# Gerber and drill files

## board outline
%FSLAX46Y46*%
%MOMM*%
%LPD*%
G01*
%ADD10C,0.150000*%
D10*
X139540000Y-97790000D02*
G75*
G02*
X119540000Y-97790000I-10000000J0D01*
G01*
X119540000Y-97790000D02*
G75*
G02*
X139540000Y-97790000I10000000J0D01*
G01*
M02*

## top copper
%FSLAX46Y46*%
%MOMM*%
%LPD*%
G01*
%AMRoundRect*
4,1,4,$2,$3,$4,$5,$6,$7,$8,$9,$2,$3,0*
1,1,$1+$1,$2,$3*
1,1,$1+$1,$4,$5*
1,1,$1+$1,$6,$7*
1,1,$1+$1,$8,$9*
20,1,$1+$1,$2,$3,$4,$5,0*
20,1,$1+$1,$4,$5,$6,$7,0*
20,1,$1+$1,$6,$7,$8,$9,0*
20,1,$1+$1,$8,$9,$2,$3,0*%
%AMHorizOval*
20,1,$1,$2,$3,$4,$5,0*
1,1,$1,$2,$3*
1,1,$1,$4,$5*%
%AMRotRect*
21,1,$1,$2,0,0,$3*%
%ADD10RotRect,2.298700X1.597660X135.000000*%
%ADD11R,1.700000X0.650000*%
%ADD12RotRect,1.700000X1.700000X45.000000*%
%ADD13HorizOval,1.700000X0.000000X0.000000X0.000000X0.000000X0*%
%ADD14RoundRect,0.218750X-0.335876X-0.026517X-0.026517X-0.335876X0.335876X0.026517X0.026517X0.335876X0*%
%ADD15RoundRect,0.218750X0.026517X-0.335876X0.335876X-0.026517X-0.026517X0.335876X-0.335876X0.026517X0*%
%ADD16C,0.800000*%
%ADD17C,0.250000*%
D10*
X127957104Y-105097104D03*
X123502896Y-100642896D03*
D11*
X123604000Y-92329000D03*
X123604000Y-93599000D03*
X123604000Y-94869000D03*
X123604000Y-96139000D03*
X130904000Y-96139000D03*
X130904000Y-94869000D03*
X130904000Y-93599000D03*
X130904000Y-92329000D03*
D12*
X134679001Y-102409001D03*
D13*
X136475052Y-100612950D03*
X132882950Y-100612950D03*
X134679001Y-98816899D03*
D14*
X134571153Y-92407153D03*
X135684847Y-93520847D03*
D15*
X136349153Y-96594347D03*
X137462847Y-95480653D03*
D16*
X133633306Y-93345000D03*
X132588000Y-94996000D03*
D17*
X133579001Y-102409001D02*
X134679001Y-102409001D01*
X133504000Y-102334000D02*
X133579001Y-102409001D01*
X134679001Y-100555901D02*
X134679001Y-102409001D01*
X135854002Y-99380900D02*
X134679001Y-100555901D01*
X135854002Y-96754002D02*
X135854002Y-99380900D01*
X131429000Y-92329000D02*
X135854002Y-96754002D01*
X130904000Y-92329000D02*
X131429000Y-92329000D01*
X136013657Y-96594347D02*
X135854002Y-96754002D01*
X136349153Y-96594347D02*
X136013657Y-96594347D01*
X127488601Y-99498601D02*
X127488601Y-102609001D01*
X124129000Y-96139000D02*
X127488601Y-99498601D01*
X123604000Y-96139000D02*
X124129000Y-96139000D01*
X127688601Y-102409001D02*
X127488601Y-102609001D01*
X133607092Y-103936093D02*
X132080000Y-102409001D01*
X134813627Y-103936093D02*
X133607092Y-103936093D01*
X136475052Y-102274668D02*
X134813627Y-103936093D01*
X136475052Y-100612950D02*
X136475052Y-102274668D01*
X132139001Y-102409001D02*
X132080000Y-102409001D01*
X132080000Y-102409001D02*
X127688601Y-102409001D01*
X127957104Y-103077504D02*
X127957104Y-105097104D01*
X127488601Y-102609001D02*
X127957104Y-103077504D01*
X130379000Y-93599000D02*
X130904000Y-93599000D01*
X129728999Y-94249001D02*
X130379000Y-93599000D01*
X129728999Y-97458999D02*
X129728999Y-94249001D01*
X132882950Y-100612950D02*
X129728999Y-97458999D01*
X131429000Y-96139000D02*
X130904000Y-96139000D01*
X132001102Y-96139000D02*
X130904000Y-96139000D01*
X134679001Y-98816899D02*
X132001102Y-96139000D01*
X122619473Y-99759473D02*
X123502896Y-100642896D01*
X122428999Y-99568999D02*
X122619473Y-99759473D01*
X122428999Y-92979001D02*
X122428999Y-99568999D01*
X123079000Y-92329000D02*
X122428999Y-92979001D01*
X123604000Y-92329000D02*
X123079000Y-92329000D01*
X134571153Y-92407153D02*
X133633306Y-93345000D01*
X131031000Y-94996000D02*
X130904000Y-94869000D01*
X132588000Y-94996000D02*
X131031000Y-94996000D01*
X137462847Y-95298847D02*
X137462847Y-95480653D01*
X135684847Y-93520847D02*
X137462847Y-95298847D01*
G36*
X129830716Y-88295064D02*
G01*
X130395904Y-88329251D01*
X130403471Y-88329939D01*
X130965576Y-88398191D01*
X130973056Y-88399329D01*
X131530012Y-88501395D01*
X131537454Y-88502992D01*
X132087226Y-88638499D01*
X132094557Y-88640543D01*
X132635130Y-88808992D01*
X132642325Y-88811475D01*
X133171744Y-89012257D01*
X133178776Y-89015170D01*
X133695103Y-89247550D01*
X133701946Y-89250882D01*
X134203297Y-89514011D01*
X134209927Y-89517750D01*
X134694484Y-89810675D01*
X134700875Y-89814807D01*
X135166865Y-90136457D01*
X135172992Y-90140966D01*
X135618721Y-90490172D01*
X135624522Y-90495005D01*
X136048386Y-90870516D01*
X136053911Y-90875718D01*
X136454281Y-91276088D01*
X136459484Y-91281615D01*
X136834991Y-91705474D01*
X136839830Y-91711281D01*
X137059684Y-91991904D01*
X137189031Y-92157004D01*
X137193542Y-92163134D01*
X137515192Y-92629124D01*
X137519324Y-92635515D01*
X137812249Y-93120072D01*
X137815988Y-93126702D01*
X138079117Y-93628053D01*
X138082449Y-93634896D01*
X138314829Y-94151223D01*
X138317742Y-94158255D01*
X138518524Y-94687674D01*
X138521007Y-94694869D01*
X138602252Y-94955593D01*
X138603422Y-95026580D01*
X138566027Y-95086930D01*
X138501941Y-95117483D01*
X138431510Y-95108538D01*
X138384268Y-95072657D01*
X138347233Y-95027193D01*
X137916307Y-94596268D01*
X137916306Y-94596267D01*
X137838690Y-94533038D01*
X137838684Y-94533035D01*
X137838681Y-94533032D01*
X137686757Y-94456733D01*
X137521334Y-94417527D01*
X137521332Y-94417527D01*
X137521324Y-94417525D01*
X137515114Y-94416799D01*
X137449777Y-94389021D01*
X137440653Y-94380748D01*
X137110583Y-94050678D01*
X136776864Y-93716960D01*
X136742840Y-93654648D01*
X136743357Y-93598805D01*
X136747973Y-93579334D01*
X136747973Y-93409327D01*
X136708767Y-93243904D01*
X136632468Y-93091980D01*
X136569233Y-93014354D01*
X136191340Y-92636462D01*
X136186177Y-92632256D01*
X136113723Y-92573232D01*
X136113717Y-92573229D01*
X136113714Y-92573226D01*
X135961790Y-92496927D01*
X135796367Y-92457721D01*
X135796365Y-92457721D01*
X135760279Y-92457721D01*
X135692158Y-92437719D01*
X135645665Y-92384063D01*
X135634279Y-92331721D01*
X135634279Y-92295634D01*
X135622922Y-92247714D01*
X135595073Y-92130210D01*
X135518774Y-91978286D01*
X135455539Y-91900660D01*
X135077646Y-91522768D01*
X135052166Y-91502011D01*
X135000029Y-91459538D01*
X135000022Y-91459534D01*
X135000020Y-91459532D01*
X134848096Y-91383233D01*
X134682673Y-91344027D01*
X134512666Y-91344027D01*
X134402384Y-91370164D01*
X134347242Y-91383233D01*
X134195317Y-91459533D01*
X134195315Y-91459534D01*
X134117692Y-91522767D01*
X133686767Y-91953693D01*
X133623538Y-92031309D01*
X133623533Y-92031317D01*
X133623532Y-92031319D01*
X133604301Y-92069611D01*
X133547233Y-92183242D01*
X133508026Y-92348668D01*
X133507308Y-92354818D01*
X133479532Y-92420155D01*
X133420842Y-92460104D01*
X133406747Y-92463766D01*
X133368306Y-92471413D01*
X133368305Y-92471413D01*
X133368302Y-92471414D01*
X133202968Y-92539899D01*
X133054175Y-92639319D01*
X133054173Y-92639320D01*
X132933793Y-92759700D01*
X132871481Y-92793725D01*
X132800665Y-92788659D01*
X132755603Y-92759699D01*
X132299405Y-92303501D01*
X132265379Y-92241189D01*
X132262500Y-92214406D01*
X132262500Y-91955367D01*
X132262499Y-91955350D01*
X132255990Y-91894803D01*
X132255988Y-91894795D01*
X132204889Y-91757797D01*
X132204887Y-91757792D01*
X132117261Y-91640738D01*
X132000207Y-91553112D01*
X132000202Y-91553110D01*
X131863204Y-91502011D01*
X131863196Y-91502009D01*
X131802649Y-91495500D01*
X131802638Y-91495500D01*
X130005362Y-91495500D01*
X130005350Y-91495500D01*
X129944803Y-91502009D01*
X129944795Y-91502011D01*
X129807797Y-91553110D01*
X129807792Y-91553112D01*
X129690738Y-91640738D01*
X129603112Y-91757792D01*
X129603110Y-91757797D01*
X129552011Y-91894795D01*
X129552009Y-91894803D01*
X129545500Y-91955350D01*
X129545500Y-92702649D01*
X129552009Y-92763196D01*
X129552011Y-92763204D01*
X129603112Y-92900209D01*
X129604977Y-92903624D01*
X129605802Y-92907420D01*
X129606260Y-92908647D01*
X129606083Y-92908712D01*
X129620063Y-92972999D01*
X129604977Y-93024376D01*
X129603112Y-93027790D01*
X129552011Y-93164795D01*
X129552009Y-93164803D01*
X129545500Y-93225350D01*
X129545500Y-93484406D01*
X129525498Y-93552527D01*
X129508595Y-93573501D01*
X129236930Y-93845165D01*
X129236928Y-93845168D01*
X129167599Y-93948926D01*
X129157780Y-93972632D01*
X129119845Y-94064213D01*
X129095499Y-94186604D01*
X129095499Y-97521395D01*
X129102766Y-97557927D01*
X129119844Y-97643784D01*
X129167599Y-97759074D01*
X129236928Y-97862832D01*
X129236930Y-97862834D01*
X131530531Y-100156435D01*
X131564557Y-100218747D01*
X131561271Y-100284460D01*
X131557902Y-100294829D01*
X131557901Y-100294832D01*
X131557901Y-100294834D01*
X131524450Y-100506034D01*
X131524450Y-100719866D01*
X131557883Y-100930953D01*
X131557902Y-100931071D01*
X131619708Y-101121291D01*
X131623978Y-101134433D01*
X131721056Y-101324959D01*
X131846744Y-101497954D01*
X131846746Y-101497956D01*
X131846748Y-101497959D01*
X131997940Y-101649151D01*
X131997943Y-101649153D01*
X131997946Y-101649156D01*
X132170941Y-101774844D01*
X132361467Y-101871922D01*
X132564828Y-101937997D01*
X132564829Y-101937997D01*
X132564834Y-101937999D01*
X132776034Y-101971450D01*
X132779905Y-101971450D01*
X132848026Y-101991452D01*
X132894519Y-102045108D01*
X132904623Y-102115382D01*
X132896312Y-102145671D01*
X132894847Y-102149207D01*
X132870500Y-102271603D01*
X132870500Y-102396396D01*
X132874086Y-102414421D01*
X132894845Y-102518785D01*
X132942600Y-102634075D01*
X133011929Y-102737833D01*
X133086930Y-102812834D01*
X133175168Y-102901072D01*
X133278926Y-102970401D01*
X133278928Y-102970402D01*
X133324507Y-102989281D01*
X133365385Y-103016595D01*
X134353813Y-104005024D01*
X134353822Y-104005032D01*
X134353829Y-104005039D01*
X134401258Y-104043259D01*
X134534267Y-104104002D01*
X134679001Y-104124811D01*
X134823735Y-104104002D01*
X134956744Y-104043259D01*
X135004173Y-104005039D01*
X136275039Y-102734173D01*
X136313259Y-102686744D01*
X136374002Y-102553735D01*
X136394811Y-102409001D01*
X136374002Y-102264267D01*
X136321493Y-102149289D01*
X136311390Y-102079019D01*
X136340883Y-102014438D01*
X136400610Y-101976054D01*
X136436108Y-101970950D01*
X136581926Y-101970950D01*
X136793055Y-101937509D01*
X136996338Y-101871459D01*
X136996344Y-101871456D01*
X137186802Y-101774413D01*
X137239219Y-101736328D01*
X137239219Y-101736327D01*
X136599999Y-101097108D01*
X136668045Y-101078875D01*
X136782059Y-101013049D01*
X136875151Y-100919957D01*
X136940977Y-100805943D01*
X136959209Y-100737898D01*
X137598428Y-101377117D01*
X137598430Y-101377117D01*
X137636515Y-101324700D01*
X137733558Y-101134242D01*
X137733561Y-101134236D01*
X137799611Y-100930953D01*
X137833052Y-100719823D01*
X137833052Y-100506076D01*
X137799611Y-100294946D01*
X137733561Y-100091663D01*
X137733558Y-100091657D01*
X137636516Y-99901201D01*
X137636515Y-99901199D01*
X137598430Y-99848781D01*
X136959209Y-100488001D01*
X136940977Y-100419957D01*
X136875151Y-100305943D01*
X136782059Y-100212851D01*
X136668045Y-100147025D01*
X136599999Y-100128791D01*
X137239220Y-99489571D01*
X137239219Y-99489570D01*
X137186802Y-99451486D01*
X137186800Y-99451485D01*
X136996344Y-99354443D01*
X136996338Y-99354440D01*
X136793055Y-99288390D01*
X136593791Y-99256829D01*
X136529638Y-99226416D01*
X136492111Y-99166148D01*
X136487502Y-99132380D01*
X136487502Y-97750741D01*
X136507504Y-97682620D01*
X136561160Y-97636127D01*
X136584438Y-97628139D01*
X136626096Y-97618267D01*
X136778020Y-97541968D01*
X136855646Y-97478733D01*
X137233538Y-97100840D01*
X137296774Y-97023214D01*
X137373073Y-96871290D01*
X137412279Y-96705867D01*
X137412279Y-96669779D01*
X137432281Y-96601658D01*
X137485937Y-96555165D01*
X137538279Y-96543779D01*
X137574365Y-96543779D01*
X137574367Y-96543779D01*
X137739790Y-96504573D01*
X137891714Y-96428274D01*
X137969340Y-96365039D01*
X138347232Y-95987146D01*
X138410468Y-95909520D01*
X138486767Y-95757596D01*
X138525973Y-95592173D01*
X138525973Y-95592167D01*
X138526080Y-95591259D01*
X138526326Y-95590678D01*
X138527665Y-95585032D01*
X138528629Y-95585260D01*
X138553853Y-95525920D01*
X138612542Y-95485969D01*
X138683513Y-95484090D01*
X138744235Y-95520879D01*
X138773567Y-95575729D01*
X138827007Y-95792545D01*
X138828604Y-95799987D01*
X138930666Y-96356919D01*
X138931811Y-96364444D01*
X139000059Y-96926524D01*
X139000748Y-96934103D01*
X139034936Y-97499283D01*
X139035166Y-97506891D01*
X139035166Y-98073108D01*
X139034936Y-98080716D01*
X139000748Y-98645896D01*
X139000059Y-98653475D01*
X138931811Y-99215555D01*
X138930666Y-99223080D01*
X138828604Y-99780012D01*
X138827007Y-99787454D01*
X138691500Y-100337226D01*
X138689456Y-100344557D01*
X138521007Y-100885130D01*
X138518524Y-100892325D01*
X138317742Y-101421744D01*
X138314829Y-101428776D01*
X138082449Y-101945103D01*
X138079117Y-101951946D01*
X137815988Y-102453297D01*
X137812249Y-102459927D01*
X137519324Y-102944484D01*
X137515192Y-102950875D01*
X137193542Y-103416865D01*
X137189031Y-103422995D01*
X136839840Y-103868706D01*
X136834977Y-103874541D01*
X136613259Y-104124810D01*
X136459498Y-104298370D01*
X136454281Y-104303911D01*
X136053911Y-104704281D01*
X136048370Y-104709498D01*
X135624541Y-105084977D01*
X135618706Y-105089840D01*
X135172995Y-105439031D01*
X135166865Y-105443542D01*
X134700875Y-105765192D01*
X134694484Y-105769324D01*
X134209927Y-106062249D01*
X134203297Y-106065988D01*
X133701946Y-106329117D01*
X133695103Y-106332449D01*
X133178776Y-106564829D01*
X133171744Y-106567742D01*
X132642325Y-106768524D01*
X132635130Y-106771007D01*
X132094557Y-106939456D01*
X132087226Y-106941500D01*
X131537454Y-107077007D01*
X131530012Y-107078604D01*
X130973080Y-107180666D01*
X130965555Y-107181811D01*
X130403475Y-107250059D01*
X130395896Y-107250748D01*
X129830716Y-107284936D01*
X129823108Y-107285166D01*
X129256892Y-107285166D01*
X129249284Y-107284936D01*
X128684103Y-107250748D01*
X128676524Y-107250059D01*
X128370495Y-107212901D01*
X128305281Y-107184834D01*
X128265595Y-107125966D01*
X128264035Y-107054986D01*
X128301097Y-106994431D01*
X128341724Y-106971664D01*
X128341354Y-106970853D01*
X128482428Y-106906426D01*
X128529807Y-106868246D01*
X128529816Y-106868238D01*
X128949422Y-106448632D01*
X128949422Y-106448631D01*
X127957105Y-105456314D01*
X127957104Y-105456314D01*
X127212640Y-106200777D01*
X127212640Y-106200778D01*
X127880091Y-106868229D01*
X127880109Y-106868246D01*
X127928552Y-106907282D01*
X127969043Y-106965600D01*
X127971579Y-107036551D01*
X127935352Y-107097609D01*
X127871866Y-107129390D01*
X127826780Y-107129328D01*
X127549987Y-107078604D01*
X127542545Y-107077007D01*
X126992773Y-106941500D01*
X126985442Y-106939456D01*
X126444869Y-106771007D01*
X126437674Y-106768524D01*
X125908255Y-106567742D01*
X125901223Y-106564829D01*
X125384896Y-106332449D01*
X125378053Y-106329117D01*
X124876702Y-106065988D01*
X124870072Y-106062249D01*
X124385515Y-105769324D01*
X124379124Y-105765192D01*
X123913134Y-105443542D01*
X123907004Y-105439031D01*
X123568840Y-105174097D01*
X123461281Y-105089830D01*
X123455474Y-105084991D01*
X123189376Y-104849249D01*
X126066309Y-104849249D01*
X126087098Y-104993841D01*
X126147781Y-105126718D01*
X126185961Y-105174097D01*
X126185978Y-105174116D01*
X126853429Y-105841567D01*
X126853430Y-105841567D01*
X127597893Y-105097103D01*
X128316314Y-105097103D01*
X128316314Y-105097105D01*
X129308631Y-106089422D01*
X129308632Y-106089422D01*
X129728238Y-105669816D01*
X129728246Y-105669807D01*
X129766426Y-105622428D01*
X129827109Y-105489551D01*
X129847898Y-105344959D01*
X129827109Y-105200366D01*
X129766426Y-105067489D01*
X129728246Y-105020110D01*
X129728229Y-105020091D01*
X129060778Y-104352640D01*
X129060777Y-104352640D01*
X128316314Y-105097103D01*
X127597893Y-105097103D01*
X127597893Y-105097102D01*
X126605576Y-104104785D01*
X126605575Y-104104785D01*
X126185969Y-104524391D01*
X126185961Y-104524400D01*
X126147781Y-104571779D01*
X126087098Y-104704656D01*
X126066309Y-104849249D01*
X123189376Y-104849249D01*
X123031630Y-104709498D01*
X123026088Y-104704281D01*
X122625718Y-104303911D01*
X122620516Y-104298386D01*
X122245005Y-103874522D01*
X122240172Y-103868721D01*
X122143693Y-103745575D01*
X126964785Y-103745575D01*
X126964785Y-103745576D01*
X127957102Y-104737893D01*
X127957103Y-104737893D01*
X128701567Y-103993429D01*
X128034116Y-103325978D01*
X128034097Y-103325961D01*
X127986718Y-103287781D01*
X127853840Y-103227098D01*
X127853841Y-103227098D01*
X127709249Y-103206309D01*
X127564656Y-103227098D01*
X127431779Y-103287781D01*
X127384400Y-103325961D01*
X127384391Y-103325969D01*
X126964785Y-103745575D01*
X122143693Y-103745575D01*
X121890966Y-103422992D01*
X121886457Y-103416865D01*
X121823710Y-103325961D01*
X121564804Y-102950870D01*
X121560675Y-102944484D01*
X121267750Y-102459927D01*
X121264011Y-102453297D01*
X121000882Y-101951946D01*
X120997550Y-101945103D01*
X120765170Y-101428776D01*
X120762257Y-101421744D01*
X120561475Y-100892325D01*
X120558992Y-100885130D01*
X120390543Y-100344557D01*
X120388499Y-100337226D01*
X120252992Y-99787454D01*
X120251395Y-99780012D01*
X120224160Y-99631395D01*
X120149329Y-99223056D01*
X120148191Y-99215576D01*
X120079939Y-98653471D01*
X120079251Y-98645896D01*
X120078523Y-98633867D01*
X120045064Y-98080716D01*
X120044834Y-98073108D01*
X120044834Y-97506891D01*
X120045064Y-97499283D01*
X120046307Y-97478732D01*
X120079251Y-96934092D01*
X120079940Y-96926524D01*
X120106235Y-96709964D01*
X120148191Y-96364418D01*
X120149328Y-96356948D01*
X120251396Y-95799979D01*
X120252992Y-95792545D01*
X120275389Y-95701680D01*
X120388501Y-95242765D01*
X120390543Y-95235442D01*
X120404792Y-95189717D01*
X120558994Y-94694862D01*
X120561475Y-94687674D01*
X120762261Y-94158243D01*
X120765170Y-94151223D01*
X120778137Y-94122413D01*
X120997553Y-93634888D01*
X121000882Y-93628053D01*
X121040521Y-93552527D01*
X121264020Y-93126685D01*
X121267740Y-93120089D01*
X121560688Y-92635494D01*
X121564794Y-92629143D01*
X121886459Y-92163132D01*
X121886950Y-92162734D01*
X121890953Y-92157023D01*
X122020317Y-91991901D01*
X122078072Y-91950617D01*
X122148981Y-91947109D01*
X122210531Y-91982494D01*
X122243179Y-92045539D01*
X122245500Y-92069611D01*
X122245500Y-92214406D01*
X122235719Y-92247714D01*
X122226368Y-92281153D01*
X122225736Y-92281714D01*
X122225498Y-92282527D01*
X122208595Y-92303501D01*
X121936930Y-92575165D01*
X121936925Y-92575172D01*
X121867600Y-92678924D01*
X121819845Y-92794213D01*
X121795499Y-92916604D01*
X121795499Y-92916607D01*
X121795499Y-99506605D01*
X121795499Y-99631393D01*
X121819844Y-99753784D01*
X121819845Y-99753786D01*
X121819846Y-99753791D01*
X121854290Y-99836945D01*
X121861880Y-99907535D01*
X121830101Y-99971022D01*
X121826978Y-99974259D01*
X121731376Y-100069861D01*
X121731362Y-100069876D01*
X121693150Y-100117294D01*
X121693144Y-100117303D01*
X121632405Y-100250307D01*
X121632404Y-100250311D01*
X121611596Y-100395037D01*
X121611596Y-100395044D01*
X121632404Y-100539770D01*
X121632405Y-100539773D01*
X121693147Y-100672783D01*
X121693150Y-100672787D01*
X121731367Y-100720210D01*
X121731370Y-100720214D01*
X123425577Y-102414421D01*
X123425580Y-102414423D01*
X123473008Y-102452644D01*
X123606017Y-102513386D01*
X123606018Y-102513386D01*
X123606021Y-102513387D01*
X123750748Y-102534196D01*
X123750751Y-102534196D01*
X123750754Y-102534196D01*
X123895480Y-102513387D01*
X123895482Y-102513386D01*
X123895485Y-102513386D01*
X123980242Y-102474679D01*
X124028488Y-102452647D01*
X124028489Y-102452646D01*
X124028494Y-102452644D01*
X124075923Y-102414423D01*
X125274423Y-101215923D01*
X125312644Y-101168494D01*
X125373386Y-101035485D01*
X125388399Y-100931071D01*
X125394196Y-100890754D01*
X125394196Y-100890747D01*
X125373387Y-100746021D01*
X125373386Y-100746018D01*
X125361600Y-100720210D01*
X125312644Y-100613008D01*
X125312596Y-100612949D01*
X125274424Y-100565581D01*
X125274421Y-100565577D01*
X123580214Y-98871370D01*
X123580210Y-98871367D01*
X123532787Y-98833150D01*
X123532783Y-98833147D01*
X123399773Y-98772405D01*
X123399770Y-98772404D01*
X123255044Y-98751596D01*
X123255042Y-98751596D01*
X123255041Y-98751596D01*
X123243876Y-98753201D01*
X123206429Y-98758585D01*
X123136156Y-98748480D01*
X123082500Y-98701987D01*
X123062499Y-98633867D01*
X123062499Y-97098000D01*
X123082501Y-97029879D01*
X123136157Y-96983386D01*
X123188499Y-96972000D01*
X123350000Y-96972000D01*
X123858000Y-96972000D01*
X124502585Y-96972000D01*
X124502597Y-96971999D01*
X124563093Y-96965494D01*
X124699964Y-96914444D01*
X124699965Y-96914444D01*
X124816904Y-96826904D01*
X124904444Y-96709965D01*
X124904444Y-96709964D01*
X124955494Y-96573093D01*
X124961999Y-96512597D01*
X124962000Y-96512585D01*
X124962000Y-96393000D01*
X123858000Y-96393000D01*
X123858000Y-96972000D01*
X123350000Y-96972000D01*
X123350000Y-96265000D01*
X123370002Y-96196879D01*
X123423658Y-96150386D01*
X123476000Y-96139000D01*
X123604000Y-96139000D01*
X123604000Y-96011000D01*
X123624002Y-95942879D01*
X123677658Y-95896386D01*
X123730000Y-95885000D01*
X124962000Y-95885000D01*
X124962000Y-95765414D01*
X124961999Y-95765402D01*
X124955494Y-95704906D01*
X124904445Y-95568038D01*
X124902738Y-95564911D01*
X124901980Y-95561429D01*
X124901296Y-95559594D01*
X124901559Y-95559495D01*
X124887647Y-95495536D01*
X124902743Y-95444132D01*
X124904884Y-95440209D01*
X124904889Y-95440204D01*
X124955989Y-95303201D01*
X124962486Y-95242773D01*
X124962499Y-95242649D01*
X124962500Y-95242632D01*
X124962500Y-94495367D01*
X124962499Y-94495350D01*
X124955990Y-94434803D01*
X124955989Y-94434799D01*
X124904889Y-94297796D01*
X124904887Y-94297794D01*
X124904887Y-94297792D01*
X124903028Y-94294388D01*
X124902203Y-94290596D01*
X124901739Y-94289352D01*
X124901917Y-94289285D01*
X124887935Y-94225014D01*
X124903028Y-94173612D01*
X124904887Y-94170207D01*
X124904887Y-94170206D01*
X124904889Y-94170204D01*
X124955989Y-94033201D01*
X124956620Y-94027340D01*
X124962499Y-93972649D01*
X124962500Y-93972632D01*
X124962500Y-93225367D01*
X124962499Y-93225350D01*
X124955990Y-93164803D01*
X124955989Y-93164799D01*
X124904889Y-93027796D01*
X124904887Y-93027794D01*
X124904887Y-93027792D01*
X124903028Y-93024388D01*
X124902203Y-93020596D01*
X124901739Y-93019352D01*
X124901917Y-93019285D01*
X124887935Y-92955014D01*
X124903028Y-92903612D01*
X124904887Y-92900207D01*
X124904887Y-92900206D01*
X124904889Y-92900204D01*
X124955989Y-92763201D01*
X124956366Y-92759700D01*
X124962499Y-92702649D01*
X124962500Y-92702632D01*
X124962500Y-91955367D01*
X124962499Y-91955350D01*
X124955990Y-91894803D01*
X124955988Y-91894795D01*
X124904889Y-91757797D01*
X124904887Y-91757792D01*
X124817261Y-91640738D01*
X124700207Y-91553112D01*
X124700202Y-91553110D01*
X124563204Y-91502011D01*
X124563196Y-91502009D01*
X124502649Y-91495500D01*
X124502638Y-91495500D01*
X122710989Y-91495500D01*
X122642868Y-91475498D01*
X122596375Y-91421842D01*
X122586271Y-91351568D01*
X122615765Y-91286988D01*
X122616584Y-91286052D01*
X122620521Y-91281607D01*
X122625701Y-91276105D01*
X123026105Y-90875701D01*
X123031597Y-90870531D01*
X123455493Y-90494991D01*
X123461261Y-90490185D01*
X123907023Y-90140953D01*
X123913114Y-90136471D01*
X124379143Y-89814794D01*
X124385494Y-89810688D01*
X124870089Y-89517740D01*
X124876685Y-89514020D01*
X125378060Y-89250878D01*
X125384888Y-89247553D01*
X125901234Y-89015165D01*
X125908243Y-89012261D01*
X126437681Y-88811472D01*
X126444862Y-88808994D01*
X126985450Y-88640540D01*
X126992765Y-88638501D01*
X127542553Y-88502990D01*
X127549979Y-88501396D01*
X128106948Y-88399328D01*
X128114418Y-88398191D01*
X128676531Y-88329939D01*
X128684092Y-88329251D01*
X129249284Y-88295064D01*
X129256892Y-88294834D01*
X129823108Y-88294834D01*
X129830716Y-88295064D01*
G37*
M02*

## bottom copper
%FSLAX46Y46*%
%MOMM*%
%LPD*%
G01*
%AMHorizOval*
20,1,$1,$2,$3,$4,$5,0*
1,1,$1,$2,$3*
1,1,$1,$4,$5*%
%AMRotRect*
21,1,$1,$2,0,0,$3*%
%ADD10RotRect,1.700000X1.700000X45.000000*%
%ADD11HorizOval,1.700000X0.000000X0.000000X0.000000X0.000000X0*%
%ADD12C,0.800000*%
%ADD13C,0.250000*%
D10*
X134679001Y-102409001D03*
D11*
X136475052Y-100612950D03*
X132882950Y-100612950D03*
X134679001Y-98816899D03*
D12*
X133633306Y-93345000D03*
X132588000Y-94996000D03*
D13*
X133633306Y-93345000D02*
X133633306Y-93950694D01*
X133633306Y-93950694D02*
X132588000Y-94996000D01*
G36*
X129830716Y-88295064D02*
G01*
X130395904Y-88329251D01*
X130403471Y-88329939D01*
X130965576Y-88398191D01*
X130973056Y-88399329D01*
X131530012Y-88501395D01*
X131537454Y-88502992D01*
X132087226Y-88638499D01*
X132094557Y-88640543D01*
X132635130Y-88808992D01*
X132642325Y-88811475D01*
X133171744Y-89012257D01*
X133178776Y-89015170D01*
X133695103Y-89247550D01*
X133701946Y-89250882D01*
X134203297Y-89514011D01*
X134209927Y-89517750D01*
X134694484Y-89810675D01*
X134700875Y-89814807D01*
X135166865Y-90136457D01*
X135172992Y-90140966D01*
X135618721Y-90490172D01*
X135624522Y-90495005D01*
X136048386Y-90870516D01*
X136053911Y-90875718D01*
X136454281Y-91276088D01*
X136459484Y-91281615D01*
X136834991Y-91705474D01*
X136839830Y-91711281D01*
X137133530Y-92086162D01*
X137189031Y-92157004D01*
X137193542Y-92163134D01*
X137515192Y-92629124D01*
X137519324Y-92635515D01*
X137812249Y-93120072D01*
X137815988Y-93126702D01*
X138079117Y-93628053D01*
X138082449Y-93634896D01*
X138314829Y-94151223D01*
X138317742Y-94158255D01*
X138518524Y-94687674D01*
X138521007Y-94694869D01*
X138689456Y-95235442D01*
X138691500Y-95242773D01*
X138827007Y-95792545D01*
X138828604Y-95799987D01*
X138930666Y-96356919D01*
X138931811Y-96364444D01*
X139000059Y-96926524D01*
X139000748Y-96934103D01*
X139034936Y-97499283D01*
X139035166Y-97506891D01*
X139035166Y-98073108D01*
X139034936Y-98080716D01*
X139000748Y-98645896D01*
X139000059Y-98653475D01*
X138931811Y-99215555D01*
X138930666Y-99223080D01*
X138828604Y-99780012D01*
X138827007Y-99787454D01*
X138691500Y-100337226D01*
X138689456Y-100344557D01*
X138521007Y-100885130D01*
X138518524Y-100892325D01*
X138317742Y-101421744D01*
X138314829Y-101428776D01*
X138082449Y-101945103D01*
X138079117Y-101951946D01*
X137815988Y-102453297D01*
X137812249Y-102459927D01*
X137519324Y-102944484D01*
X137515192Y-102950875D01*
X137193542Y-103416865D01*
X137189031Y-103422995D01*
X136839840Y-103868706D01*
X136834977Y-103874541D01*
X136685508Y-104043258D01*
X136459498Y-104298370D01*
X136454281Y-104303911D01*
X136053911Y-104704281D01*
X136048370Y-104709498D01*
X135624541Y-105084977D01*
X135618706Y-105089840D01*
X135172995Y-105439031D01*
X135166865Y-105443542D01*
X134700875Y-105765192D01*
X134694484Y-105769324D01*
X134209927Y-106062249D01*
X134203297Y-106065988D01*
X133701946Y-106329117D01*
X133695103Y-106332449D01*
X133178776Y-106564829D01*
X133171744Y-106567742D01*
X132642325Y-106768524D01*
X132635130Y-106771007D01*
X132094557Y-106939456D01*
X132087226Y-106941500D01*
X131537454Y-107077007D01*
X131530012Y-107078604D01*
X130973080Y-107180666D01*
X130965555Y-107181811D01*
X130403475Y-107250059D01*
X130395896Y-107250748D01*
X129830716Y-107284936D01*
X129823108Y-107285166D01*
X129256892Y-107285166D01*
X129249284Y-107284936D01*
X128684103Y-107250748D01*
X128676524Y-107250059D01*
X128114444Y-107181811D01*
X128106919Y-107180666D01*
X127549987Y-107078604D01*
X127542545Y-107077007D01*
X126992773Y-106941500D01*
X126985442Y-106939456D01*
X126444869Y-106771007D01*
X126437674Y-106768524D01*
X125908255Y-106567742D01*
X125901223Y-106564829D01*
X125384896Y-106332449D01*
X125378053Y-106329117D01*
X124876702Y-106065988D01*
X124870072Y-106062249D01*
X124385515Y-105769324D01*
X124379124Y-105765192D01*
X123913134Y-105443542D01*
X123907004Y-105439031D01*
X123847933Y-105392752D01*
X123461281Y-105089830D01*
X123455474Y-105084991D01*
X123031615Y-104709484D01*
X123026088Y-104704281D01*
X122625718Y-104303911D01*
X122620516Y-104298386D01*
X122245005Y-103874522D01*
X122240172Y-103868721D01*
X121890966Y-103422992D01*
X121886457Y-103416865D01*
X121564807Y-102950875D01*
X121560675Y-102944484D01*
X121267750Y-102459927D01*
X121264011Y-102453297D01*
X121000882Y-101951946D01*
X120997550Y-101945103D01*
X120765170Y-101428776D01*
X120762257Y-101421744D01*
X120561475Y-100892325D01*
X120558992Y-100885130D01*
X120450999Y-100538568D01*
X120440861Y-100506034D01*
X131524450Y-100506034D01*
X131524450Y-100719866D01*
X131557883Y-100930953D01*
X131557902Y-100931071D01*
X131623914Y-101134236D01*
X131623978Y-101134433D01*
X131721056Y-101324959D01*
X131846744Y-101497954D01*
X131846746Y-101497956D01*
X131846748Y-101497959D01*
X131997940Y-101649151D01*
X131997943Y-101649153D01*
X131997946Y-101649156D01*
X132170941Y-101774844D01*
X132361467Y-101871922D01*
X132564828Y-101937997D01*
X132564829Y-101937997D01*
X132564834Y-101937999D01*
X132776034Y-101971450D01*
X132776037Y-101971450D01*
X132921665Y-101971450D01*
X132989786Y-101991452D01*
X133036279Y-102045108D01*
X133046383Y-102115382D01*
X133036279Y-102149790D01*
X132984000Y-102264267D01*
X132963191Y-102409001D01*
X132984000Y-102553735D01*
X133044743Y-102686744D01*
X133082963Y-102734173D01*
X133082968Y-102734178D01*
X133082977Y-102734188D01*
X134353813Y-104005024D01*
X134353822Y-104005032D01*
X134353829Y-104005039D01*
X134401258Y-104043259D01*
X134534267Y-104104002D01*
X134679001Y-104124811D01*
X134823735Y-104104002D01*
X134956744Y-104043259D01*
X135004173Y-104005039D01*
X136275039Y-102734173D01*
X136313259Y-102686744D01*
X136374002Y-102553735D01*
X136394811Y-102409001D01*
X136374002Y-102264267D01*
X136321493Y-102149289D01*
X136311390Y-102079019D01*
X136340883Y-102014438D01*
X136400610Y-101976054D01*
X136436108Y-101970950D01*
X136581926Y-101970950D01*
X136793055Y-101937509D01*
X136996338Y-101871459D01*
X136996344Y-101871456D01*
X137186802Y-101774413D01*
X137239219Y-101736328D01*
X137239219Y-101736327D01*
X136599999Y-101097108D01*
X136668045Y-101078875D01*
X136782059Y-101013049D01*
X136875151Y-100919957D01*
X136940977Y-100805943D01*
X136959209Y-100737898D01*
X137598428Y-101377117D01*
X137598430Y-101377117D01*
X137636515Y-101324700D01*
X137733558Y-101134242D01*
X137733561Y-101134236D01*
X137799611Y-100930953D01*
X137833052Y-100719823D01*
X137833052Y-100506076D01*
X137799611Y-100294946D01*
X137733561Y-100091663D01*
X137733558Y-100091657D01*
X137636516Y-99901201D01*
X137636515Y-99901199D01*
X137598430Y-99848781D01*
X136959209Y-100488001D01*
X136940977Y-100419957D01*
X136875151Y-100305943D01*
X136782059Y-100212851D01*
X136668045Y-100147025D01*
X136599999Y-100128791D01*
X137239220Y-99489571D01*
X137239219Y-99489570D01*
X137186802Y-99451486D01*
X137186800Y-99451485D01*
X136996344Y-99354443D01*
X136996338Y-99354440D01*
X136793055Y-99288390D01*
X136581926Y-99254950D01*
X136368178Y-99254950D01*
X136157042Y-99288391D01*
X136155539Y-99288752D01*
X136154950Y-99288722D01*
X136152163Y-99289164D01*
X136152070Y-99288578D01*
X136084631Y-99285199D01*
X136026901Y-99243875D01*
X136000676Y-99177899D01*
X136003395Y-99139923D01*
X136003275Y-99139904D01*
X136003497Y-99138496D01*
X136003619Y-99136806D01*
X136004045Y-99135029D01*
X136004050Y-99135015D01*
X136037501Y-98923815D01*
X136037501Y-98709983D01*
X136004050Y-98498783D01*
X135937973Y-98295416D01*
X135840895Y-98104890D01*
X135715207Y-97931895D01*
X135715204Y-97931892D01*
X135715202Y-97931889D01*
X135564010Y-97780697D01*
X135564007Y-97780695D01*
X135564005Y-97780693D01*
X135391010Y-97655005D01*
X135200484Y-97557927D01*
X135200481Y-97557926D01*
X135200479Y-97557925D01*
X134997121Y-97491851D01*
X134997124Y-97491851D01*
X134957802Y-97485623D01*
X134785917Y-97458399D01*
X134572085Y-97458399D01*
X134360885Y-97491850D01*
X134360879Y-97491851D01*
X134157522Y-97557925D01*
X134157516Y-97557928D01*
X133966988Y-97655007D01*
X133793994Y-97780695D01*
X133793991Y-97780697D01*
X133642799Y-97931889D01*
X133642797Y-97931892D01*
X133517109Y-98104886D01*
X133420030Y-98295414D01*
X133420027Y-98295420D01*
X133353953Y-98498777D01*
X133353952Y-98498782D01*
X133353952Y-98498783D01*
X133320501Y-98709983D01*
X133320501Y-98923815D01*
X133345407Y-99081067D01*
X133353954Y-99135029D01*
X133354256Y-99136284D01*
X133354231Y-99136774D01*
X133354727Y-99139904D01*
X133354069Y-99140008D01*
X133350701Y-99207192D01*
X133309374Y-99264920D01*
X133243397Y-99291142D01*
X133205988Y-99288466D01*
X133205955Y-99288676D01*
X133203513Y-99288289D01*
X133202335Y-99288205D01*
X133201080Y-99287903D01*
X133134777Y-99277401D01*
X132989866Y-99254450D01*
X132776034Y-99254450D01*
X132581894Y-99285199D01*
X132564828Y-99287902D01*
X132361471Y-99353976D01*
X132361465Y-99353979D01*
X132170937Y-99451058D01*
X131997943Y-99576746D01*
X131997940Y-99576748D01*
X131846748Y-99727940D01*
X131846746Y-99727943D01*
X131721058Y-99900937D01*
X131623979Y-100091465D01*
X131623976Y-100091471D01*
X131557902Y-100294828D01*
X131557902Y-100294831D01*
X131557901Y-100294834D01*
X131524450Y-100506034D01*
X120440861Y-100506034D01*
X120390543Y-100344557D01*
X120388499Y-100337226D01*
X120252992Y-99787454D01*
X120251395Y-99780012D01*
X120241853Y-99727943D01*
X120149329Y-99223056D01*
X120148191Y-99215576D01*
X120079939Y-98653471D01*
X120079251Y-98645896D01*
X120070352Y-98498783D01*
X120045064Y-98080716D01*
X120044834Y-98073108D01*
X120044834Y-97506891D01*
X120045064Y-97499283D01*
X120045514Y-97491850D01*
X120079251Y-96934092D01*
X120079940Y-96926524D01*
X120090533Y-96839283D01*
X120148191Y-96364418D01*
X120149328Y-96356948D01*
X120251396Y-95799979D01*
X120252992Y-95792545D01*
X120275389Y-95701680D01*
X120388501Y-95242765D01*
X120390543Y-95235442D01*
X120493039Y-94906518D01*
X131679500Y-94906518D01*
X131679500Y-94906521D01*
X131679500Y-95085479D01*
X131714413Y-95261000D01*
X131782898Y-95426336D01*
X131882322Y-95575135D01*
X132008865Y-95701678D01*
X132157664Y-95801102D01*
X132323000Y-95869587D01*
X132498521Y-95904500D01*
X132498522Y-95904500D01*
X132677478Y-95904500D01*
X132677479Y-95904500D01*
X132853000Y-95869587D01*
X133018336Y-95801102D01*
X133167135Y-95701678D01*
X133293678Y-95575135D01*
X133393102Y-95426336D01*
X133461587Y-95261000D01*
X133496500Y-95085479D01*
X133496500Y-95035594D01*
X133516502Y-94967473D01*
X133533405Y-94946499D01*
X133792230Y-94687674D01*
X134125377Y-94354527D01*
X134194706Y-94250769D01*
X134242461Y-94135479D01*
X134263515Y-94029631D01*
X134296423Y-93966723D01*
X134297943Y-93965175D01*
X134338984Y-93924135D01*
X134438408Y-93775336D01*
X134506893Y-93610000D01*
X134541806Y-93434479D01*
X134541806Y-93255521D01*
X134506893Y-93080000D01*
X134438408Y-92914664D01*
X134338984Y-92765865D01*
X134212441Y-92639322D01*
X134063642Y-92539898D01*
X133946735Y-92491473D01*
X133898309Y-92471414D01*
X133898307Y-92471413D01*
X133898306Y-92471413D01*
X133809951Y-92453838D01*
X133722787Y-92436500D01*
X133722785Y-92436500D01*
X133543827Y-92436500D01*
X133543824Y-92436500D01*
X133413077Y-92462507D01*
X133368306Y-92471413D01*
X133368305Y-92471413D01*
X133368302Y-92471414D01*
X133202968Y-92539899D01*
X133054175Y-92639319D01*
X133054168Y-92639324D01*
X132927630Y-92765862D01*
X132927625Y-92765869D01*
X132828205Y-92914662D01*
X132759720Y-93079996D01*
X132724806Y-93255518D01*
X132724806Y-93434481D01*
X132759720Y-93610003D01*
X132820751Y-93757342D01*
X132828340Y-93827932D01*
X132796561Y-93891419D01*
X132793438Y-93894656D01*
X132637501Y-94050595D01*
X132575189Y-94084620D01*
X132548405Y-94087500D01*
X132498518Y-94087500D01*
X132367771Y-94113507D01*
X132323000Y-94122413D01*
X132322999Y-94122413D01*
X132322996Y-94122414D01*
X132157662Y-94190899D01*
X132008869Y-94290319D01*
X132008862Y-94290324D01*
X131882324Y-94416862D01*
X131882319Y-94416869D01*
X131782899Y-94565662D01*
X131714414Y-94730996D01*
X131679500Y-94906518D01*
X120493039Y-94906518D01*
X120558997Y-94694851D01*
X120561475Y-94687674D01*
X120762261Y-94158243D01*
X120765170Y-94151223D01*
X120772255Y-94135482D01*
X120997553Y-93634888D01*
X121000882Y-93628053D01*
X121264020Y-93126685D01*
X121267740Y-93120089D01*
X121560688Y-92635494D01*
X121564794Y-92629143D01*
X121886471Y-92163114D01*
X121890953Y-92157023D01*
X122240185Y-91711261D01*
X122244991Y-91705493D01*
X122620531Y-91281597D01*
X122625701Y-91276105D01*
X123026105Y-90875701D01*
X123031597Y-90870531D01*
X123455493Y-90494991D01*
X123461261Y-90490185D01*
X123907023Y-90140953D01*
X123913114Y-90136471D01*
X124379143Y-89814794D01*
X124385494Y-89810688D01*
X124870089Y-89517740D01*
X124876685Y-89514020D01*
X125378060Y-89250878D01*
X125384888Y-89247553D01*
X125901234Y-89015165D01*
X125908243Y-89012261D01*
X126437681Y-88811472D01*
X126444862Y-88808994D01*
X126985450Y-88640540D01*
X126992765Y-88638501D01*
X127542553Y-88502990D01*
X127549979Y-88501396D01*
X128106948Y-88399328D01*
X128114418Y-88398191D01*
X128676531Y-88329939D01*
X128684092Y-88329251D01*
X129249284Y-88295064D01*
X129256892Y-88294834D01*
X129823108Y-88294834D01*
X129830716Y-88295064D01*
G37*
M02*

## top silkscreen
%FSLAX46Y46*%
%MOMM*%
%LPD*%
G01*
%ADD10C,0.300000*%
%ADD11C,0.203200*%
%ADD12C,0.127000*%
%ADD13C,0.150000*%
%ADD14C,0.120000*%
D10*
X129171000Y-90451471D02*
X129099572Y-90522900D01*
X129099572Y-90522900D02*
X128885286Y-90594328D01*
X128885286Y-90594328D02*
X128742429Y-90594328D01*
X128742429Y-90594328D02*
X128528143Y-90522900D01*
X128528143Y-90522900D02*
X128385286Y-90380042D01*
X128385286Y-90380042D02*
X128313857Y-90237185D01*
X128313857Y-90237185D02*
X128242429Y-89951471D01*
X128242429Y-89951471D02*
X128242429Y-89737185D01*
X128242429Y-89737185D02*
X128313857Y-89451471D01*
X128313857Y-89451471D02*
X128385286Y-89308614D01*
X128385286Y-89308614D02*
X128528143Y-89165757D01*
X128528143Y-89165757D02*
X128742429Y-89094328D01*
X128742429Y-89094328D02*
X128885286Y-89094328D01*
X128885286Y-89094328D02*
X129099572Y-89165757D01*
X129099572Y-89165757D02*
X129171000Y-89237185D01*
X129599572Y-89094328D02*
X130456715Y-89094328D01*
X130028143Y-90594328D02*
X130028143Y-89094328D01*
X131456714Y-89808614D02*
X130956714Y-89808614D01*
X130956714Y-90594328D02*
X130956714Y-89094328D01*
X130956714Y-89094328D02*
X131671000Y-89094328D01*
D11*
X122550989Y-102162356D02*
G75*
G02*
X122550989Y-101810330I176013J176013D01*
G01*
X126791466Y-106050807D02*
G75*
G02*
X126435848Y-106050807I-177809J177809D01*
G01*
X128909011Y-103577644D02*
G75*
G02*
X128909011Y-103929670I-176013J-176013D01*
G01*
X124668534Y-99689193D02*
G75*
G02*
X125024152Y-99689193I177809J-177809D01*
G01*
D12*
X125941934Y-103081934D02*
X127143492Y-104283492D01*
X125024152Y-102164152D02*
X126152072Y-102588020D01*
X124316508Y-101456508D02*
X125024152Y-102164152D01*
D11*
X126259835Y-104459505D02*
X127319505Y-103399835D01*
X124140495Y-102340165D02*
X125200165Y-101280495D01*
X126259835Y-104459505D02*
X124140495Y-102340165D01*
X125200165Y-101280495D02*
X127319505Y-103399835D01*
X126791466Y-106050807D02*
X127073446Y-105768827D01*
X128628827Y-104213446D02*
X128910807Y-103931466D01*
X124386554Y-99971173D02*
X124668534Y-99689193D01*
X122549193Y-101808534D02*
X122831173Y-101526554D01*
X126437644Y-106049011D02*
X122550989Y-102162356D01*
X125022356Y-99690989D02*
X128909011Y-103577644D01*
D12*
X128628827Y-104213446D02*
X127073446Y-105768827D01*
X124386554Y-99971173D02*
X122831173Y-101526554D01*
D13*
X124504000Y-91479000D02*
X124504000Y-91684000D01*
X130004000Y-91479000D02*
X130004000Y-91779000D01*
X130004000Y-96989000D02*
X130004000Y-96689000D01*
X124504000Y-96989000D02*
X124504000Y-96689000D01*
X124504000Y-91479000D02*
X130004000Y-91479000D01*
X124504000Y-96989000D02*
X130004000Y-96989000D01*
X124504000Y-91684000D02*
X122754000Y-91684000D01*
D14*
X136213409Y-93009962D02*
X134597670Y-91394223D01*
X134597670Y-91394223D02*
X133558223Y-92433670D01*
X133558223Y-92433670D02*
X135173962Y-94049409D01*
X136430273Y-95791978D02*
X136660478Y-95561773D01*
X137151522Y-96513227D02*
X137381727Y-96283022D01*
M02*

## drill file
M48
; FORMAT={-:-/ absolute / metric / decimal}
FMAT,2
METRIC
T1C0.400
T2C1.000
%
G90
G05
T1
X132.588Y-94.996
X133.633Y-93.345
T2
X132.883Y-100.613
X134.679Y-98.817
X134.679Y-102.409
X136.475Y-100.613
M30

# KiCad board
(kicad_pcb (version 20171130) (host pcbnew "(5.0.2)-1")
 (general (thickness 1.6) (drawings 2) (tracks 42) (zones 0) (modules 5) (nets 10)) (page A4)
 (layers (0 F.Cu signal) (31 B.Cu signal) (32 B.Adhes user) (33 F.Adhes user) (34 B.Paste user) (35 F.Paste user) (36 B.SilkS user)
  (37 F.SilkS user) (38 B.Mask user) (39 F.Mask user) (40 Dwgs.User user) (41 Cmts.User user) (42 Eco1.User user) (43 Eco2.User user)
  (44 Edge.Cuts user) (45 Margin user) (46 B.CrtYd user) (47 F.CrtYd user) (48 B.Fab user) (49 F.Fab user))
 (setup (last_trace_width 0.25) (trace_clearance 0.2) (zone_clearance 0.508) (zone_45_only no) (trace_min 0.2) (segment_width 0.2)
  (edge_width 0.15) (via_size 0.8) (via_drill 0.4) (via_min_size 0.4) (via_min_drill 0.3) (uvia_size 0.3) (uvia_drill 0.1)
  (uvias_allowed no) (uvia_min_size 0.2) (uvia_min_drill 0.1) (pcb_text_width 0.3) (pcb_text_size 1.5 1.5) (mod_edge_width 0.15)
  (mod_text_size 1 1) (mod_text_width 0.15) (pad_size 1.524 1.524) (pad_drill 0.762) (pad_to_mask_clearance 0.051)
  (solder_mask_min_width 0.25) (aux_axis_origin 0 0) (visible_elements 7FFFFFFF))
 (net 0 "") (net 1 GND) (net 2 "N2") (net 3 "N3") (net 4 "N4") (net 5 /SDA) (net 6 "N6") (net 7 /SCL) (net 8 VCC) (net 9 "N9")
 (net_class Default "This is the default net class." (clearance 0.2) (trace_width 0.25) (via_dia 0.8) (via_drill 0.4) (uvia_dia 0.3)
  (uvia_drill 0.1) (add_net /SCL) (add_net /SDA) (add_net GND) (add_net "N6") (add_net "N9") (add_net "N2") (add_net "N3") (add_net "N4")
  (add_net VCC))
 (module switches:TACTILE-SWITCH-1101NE (layer F.Cu) (at 125.73 102.87 315)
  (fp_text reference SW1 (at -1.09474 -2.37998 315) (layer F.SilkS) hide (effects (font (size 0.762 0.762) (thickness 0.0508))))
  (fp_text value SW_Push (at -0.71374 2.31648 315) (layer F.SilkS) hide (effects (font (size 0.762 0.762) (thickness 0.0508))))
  (fp_arc (start -2.74828 1.4986) (end -2.74828 1.74752) (angle 90) (layer F.SilkS) (width 0.2032))
  (fp_arc (start 2.74828 1.4986) (end 2.99974 1.4986) (angle 90) (layer F.SilkS) (width 0.2032))
  (fp_arc (start 2.74828 -1.4986) (end 2.74828 -1.74752) (angle 90) (layer F.SilkS) (width 0.2032))
  (fp_arc (start -2.74828 -1.4986) (end -2.99974 -1.4986) (angle 90) (layer F.SilkS) (width 0.2032))
  (fp_line (start 0.29972 0) (end 1.99898 0) (layer F.SilkS) (width 0.127))
  (fp_line (start -0.99822 0) (end 0.09906 -0.49784) (layer F.SilkS) (width 0.127))
  (fp_line (start -1.99898 0) (end -0.99822 0) (layer F.SilkS) (width 0.127))
  (fp_line (start 1.4986 0.7493) (end 1.4986 -0.7493) (layer F.SilkS) (width 0.2032))
  (fp_line (start -1.4986 0.7493) (end -1.4986 -0.7493) (layer F.SilkS) (width 0.2032))
  (fp_line (start 1.4986 0.7493) (end -1.4986 0.7493) (layer F.SilkS) (width 0.2032))
  (fp_line (start -1.4986 -0.7493) (end 1.4986 -0.7493) (layer F.SilkS) (width 0.2032))
  (fp_line (start 2.99974 1.4986) (end 2.99974 1.09982) (layer F.SilkS) (width 0.2032))
  (fp_line (start 2.99974 -1.09982) (end 2.99974 -1.4986) (layer F.SilkS) (width 0.2032))
  (fp_line (start -2.99974 -1.09982) (end -2.99974 -1.4986) (layer F.SilkS) (width 0.2032))
  (fp_line (start -2.99974 1.4986) (end -2.99974 1.09982) (layer F.SilkS) (width 0.2032))
  (fp_line (start 2.74828 1.74752) (end -2.74828 1.74752) (layer F.SilkS) (width 0.2032))
  (fp_line (start -2.74828 -1.74752) (end 2.74828 -1.74752) (layer F.SilkS) (width 0.2032))
  (fp_line (start 2.99974 -1.09982) (end 2.99974 1.09982) (layer F.SilkS) (width 0.127))
  (fp_line (start -2.99974 -1.09982) (end -2.99974 1.09982) (layer F.SilkS) (width 0.127))
  (pad 2 smd rect (at 3.149601 0 135) (size 2.2987 1.59766) (layers F.Cu F.Paste F.Mask) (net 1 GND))
  (pad 1 smd rect (at -3.149601 0 135) (size 2.2987 1.59766) (layers F.Cu F.Paste F.Mask) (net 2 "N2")))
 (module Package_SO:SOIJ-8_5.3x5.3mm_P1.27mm (layer F.Cu) (at 127.254 94.234)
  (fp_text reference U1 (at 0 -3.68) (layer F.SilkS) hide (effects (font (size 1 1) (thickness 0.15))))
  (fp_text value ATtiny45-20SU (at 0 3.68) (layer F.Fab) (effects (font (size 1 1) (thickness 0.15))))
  (fp_line (start -2.75 -2.755) (end -2.75 -2.55) (layer F.SilkS) (width 0.15))
  (fp_line (start 2.75 -2.755) (end 2.75 -2.455) (layer F.SilkS) (width 0.15))
  (fp_line (start 2.75 2.755) (end 2.75 2.455) (layer F.SilkS) (width 0.15))
  (fp_line (start -2.75 2.755) (end -2.75 2.455) (layer F.SilkS) (width 0.15))
  (fp_line (start -2.75 -2.755) (end 2.75 -2.755) (layer F.SilkS) (width 0.15))
  (fp_line (start -2.75 2.755) (end 2.75 2.755) (layer F.SilkS) (width 0.15))
  (fp_line (start -2.75 -2.55) (end -4.5 -2.55) (layer F.SilkS) (width 0.15))
  (pad 1 smd rect (at -3.65 -1.905) (size 1.7 0.65) (layers F.Cu F.Paste F.Mask) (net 2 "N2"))
  (pad 2 smd rect (at -3.65 -0.635) (size 1.7 0.65) (layers F.Cu F.Paste F.Mask) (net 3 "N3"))
  (pad 3 smd rect (at -3.65 0.635) (size 1.7 0.65) (layers F.Cu F.Paste F.Mask) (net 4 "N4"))
  (pad 4 smd rect (at -3.65 1.905) (size 1.7 0.65) (layers F.Cu F.Paste F.Mask) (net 1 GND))
  (pad 5 smd rect (at 3.65 1.905) (size 1.7 0.65) (layers F.Cu F.Paste F.Mask) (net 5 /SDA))
  (pad 6 smd rect (at 3.65 0.635) (size 1.7 0.65) (layers F.Cu F.Paste F.Mask) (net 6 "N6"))
  (pad 7 smd rect (at 3.65 -0.635) (size 1.7 0.65) (layers F.Cu F.Paste F.Mask) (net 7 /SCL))
  (pad 8 smd rect (at 3.65 -1.905) (size 1.7 0.65) (layers F.Cu F.Paste F.Mask) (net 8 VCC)))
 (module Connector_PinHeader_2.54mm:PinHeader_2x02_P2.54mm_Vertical (layer B.Cu) (at 134.679001 102.409001 45)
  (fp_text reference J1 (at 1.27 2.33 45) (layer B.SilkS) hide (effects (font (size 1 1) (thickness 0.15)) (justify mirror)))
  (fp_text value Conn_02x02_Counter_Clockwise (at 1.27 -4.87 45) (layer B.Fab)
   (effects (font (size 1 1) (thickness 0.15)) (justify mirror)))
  (pad 1 thru_hole rect (at 0 0 45) (size 1.7 1.7) (drill 1) (layers *.Cu *.Mask) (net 8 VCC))
  (pad 2 thru_hole oval (at 2.54 0 45) (size 1.7 1.7) (drill 1) (layers *.Cu *.Mask) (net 1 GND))
  (pad 3 thru_hole oval (at 0 -2.54 45) (size 1.7 1.7) (drill 1) (layers *.Cu *.Mask) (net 7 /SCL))
  (pad 4 thru_hole oval (at 2.54 -2.54 45) (size 1.7 1.7) (drill 1) (layers *.Cu *.Mask) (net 5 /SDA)))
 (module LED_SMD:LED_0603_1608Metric (layer F.Cu) (at 135.128 92.964 315)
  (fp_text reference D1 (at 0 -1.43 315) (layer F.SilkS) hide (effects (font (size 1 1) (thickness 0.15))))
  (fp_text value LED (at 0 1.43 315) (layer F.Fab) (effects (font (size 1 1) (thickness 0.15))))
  (fp_line (start 0.8 -0.735) (end -1.485 -0.735) (layer F.SilkS) (width 0.12))
  (fp_line (start -1.485 -0.735) (end -1.485 0.735) (layer F.SilkS) (width 0.12))
  (fp_line (start -1.485 0.735) (end 0.8 0.735) (layer F.SilkS) (width 0.12))
  (pad 1 smd roundrect (at -0.787501 0 315) (size 0.875 0.95) (layers F.Cu F.Paste F.Mask) (roundrect_rratio 0.25) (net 6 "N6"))
  (pad 2 smd roundrect (at 0.787501 0 315) (size 0.875 0.95) (layers F.Cu F.Paste F.Mask) (roundrect_rratio 0.25) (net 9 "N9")))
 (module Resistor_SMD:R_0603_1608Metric (layer F.Cu) (at 136.906 96.0375 45)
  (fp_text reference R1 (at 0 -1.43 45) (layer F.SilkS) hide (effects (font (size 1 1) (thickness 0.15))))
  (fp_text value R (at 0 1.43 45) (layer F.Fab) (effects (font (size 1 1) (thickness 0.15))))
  (fp_line (start -0.162779 -0.51) (end 0.162779 -0.51) (layer F.SilkS) (width 0.12))
  (fp_line (start -0.162779 0.51) (end 0.162779 0.51) (layer F.SilkS) (width 0.12))
  (pad 1 smd roundrect (at -0.7875 0 45) (size 0.875 0.95) (layers F.Cu F.Paste F.Mask) (roundrect_rratio 0.25) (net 8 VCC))
  (pad 2 smd roundrect (at 0.7875 0 45) (size 0.875 0.95) (layers F.Cu F.Paste F.Mask) (roundrect_rratio 0.25) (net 9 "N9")))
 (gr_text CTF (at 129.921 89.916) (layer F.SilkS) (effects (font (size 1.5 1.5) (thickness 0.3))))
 (gr_circle (center 129.54 97.79) (end 139.54 97.79) (layer Edge.Cuts) (width 0.15))
 (segment (start 133.579001 102.409001) (end 134.679001 102.409001) (width 0.25) (layer F.Cu) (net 8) (status 30))
 (segment (start 133.504 102.334) (end 133.579001 102.409001) (width 0.25) (layer F.Cu) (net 8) (status 20))
 (segment (start 134.679001 100.555901) (end 134.679001 102.409001) (width 0.25) (layer F.Cu) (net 8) (status 20))
 (segment (start 135.854002 99.3809) (end 134.679001 100.555901) (width 0.25) (layer F.Cu) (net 8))
 (segment (start 135.854002 96.754002) (end 135.854002 99.3809) (width 0.25) (layer F.Cu) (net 8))
 (segment (start 131.429 92.329) (end 135.854002 96.754002) (width 0.25) (layer F.Cu) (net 8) (status 10))
 (segment (start 130.904 92.329) (end 131.429 92.329) (width 0.25) (layer F.Cu) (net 8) (status 30))
 (segment (start 136.013657 96.594347) (end 135.854002 96.754002) (width 0.25) (layer F.Cu) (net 8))
 (segment (start 136.349153 96.594347) (end 136.013657 96.594347) (width 0.25) (layer F.Cu) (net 8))
 (segment (start 127.488601 99.498601) (end 127.488601 102.609001) (width 0.25) (layer F.Cu) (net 1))
 (segment (start 124.129 96.139) (end 127.488601 99.498601) (width 0.25) (layer F.Cu) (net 1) (status 10))
 (segment (start 123.604 96.139) (end 124.129 96.139) (width 0.25) (layer F.Cu) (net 1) (status 30))
 (segment (start 127.688601 102.409001) (end 127.488601 102.609001) (width 0.25) (layer F.Cu) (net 1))
 (segment (start 133.607092 103.936093) (end 132.08 102.409001) (width 0.25) (layer F.Cu) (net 1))
 (segment (start 134.813627 103.936093) (end 133.607092 103.936093) (width 0.25) (layer F.Cu) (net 1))
 (segment (start 136.475052 102.274668) (end 134.813627 103.936093) (width 0.25) (layer F.Cu) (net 1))
 (segment (start 136.475052 100.61295) (end 136.475052 102.274668) (width 0.25) (layer F.Cu) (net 1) (status 10))
 (segment (start 132.139001 102.409001) (end 132.08 102.409001) (width 0.25) (layer F.Cu) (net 1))
 (segment (start 132.08 102.409001) (end 127.688601 102.409001) (width 0.25) (layer F.Cu) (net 1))
 (segment (start 127.957104 103.077504) (end 127.957104 105.097104) (width 0.25) (layer F.Cu) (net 1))
 (segment (start 127.488601 102.609001) (end 127.957104 103.077504) (width 0.25) (layer F.Cu) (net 1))
 (segment (start 130.379 93.599) (end 130.904 93.599) (width 0.25) (layer F.Cu) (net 7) (status 30))
 (segment (start 129.728999 94.249001) (end 130.379 93.599) (width 0.25) (layer F.Cu) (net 7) (status 20))
 (segment (start 129.728999 97.458999) (end 129.728999 94.249001) (width 0.25) (layer F.Cu) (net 7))
 (segment (start 132.88295 100.61295) (end 129.728999 97.458999) (width 0.25) (layer F.Cu) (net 7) (status 10))
 (segment (start 131.429 96.139) (end 130.904 96.139) (width 0.25) (layer F.Cu) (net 5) (status 30))
 (segment (start 132.001102 96.139) (end 130.904 96.139) (width 0.25) (layer F.Cu) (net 5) (status 20))
 (segment (start 134.679001 98.816899) (end 132.001102 96.139) (width 0.25) (layer F.Cu) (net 5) (status 10))
 (segment (start 122.619473 99.759473) (end 123.502896 100.642896) (width 0.25) (layer F.Cu) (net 2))
 (segment (start 122.428999 99.568999) (end 122.619473 99.759473) (width 0.25) (layer F.Cu) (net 2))
 (segment (start 122.428999 92.979001) (end 122.428999 99.568999) (width 0.25) (layer F.Cu) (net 2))
 (segment (start 123.079 92.329) (end 122.428999 92.979001) (width 0.25) (layer F.Cu) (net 2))
 (segment (start 123.604 92.329) (end 123.079 92.329) (width 0.25) (layer F.Cu) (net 2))
 (segment (start 134.571153 92.407153) (end 133.633306 93.345) (width 0.25) (layer F.Cu) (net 6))
 (via (at 133.633306 93.345) (size 0.8) (drill 0.4) (layers F.Cu B.Cu) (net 6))
 (segment (start 133.633306 93.345) (end 133.633306 93.950694) (width 0.25) (layer B.Cu) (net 6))
 (via (at 132.588 94.996) (size 0.8) (drill 0.4) (layers F.Cu B.Cu) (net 6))
 (segment (start 133.633306 93.950694) (end 132.588 94.996) (width 0.25) (layer B.Cu) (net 6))
 (segment (start 131.031 94.996) (end 130.904 94.869) (width 0.25) (layer F.Cu) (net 6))
 (segment (start 132.588 94.996) (end 131.031 94.996) (width 0.25) (layer F.Cu) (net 6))
 (segment (start 137.462847 95.298847) (end 137.462847 95.480653) (width 0.25) (layer F.Cu) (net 9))
 (segment (start 135.684847 93.520847) (end 137.462847 95.298847) (width 0.25) (layer F.Cu) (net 9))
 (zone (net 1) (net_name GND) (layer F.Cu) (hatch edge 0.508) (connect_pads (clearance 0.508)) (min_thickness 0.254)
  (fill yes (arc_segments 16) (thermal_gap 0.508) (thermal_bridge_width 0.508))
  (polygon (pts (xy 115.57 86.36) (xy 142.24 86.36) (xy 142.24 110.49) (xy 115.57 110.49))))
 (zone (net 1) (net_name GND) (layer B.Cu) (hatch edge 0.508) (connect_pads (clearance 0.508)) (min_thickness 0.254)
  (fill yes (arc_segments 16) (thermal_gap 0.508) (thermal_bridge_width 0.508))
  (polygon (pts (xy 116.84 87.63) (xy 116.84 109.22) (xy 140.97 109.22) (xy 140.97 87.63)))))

